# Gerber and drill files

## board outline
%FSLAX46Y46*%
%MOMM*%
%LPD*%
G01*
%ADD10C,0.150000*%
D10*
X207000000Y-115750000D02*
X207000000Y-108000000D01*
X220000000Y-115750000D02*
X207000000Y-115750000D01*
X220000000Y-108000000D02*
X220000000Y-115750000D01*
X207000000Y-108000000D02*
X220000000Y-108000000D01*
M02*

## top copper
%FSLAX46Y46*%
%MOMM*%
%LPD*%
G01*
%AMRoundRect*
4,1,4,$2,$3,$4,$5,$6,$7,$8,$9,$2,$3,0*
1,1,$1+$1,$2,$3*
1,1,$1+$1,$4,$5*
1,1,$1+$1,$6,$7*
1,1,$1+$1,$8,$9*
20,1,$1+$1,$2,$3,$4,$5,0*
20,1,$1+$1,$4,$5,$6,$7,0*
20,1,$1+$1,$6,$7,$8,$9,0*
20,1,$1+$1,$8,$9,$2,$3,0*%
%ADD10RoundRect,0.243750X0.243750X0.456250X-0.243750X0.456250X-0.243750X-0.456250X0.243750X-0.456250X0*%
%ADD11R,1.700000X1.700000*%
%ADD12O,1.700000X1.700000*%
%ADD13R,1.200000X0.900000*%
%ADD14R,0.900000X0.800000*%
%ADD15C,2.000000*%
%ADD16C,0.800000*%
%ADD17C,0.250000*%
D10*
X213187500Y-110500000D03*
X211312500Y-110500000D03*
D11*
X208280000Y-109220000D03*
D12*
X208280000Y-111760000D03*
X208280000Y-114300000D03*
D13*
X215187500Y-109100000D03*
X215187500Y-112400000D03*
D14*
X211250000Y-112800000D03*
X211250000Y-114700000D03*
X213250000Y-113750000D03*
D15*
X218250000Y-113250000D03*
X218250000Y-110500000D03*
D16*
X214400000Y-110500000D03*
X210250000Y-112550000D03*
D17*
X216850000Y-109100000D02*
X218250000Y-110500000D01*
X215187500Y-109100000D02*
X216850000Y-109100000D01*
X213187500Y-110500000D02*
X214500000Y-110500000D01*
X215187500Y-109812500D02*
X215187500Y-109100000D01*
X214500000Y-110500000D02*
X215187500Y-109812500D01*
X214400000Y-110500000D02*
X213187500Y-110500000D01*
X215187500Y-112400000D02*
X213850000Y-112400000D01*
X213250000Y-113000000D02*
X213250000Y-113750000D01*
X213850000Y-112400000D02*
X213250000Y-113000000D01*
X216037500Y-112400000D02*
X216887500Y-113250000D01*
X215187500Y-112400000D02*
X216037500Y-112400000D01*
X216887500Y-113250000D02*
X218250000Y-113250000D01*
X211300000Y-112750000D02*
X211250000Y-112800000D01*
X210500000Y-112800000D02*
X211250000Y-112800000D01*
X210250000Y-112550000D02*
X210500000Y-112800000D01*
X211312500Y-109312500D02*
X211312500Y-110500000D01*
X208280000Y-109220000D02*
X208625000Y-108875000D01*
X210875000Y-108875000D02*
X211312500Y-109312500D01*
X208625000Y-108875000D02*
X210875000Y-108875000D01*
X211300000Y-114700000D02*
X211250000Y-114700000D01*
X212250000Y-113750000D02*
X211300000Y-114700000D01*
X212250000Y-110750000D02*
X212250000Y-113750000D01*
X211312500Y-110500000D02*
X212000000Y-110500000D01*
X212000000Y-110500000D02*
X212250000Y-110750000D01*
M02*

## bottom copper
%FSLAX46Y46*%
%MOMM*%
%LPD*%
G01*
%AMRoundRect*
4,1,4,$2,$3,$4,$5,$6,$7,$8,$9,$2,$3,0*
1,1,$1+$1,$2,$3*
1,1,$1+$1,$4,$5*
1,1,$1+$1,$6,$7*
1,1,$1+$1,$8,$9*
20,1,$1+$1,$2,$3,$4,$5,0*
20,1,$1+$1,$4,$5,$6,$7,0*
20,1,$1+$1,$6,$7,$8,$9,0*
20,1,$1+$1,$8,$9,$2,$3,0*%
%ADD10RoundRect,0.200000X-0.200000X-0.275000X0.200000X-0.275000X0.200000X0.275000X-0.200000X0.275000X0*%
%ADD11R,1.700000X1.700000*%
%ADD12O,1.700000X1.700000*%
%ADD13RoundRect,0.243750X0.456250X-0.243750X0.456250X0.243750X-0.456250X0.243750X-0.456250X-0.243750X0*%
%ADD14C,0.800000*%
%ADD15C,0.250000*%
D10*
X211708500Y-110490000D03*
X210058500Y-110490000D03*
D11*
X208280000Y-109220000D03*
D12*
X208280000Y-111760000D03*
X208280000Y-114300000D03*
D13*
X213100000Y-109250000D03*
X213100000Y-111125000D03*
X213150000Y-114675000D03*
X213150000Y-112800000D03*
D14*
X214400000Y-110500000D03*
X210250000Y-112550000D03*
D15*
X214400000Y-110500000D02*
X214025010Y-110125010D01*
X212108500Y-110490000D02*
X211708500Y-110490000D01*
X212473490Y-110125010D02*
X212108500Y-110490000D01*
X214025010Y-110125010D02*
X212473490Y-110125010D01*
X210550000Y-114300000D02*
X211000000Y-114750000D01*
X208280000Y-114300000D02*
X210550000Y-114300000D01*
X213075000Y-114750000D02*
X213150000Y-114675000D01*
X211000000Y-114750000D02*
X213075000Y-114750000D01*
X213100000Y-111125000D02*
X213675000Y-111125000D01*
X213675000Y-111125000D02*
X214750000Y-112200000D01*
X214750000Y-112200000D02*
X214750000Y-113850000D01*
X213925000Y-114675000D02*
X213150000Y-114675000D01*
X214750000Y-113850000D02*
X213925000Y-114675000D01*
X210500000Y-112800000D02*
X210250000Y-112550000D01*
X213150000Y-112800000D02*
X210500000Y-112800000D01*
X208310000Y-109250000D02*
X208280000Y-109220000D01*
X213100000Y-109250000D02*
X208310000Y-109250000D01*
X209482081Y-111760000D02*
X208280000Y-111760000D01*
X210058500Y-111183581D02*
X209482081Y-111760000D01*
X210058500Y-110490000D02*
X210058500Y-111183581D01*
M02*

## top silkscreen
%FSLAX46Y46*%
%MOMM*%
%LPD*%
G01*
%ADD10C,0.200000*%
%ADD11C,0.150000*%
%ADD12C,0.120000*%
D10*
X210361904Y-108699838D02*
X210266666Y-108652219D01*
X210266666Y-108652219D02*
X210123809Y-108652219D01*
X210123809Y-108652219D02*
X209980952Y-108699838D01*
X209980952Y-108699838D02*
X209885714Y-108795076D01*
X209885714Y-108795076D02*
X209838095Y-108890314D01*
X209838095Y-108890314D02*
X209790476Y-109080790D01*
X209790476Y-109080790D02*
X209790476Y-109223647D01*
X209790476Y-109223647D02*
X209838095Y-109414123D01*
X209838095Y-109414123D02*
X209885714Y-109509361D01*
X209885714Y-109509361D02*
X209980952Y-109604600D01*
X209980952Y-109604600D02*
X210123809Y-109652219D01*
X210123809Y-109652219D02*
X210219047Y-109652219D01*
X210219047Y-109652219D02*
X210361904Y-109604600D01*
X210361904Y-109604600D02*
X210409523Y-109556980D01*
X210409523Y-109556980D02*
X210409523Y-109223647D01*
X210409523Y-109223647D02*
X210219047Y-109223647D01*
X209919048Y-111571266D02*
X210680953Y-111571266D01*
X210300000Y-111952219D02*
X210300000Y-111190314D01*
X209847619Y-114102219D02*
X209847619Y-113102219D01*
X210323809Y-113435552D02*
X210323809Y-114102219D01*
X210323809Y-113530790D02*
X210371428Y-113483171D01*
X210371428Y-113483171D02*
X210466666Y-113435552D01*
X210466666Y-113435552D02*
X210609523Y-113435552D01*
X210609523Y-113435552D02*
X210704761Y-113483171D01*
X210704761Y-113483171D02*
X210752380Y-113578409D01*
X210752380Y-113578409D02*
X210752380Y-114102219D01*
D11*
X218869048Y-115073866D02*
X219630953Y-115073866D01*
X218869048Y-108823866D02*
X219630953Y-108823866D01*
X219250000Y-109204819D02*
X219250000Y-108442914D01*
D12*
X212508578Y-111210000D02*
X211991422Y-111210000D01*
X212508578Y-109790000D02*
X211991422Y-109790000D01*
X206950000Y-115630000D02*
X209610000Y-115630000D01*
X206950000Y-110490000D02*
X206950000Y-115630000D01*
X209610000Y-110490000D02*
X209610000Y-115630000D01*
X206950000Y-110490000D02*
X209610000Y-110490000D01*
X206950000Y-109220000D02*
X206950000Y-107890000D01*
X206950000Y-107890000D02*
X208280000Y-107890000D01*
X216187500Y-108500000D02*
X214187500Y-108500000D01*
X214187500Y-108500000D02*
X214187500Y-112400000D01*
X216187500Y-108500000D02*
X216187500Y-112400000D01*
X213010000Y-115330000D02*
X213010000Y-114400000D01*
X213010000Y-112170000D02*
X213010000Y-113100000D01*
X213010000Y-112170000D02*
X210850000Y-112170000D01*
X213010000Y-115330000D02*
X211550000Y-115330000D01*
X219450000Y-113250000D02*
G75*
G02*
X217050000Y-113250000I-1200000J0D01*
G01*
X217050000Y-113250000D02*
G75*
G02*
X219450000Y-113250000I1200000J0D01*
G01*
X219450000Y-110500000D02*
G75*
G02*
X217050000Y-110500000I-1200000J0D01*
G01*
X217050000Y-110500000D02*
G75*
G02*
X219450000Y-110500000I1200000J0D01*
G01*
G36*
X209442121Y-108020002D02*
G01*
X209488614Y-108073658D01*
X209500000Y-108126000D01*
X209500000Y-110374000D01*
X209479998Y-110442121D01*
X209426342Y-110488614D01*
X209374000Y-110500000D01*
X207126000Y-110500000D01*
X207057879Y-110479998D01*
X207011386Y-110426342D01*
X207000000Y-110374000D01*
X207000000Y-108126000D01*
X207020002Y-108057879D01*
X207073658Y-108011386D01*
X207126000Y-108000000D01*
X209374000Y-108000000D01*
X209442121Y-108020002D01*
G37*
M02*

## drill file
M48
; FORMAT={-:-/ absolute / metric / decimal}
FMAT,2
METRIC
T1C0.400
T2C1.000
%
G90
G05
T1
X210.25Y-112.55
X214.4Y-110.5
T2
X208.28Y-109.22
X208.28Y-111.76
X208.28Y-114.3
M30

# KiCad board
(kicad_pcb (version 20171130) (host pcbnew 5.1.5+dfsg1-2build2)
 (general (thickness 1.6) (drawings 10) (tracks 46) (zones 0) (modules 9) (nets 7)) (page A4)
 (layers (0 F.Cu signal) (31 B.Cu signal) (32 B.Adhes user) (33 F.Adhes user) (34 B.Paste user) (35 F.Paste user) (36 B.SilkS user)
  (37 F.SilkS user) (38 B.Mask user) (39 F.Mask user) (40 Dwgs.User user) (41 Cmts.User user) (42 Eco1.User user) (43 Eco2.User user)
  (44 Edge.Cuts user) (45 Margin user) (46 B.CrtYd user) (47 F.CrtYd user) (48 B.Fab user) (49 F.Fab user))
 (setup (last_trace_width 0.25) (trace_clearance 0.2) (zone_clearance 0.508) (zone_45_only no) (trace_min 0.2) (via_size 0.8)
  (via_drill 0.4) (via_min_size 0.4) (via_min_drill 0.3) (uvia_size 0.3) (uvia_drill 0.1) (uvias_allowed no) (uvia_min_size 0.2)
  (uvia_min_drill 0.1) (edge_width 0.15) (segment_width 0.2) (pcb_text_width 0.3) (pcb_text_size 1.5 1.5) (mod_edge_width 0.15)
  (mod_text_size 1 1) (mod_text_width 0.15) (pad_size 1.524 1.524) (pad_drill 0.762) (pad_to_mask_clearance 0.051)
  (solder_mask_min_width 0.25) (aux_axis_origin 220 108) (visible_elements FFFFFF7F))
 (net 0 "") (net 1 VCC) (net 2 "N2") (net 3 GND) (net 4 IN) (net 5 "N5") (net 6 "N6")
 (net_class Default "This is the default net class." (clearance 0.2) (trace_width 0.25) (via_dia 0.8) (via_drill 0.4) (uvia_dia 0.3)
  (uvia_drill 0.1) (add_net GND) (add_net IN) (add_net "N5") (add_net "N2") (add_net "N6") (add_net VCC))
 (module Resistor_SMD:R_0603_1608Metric (layer B.Cu) (at 210.8835 110.49)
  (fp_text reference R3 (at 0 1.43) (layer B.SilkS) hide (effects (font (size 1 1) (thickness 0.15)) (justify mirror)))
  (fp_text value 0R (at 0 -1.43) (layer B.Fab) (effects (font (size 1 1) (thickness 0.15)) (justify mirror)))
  (pad 2 smd roundrect (at 0.825 0) (size 0.8 0.95) (layers B.Cu B.Paste B.Mask) (roundrect_rratio 0.25) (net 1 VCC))
  (pad 1 smd roundrect (at -0.825 0) (size 0.8 0.95) (layers B.Cu B.Paste B.Mask) (roundrect_rratio 0.25) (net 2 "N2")))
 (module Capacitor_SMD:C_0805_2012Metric (layer F.Cu) (at 212.25 110.5 180)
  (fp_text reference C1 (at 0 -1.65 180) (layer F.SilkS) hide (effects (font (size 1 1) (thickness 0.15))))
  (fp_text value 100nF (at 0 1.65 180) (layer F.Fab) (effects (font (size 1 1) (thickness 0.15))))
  (fp_line (start -0.258578 -0.71) (end 0.258578 -0.71) (layer F.SilkS) (width 0.12))
  (fp_line (start -0.258578 0.71) (end 0.258578 0.71) (layer F.SilkS) (width 0.12))
  (pad 1 smd roundrect (at -0.9375 0 180) (size 0.975 1.4) (layers F.Cu F.Paste F.Mask) (roundrect_rratio 0.25) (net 1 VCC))
  (pad 2 smd roundrect (at 0.9375 0 180) (size 0.975 1.4) (layers F.Cu F.Paste F.Mask) (roundrect_rratio 0.25) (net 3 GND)))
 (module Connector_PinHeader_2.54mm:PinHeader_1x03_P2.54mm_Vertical (layer F.Cu) (at 208.28 109.22)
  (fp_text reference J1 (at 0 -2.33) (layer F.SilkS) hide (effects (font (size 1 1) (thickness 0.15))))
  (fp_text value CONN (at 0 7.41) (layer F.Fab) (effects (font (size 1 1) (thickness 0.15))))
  (fp_line (start -1.33 6.41) (end 1.33 6.41) (layer F.SilkS) (width 0.12))
  (fp_line (start -1.33 1.27) (end -1.33 6.41) (layer F.SilkS) (width 0.12))
  (fp_line (start 1.33 1.27) (end 1.33 6.41) (layer F.SilkS) (width 0.12))
  (fp_line (start -1.33 1.27) (end 1.33 1.27) (layer F.SilkS) (width 0.12))
  (fp_line (start -1.33 0) (end -1.33 -1.33) (layer F.SilkS) (width 0.12))
  (fp_line (start -1.33 -1.33) (end 0 -1.33) (layer F.SilkS) (width 0.12))
  (pad 1 thru_hole rect (at 0 0) (size 1.7 1.7) (drill 1) (layers *.Cu *.Mask) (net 3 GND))
  (pad 2 thru_hole oval (at 0 2.54) (size 1.7 1.7) (drill 1) (layers *.Cu *.Mask) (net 2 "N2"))
  (pad 3 thru_hole oval (at 0 5.08) (size 1.7 1.7) (drill 1) (layers *.Cu *.Mask) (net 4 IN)))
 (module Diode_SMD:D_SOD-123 (layer F.Cu) (at 215.1875 110.75 270)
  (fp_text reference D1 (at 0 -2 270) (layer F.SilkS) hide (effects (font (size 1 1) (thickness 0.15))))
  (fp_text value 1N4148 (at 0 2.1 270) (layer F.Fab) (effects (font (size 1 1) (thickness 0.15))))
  (fp_line (start -2.25 -1) (end -2.25 1) (layer F.SilkS) (width 0.12))
  (fp_line (start -2.25 1) (end 1.65 1) (layer F.SilkS) (width 0.12))
  (fp_line (start -2.25 -1) (end 1.65 -1) (layer F.SilkS) (width 0.12))
  (pad 1 smd rect (at -1.65 0 270) (size 0.9 1.2) (layers F.Cu F.Paste F.Mask) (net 1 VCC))
  (pad 2 smd rect (at 1.65 0 270) (size 0.9 1.2) (layers F.Cu F.Paste F.Mask) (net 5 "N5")))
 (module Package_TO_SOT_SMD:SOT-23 (layer F.Cu) (at 212.25 113.75)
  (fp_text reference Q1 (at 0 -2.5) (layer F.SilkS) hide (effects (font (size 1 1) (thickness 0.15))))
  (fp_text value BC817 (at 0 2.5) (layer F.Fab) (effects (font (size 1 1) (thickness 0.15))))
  (fp_line (start 0.76 1.58) (end 0.76 0.65) (layer F.SilkS) (width 0.12))
  (fp_line (start 0.76 -1.58) (end 0.76 -0.65) (layer F.SilkS) (width 0.12))
  (fp_line (start 0.76 -1.58) (end -1.4 -1.58) (layer F.SilkS) (width 0.12))
  (fp_line (start 0.76 1.58) (end -0.7 1.58) (layer F.SilkS) (width 0.12))
  (pad 1 smd rect (at -1 -0.95) (size 0.9 0.8) (layers F.Cu F.Paste F.Mask) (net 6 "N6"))
  (pad 2 smd rect (at -1 0.95) (size 0.9 0.8) (layers F.Cu F.Paste F.Mask) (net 3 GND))
  (pad 3 smd rect (at 1 0) (size 0.9 0.8) (layers F.Cu F.Paste F.Mask) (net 5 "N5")))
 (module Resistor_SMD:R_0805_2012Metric (layer B.Cu) (at 213.1 110.1875 90)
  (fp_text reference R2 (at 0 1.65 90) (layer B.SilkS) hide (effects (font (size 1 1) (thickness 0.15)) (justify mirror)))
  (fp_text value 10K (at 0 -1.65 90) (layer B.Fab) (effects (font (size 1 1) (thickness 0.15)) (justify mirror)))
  (pad 2 smd roundrect (at 0.9375 0 90) (size 0.975 1.4) (layers B.Cu B.Paste B.Mask) (roundrect_rratio 0.25) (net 3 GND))
  (pad 1 smd roundrect (at -0.9375 0 90) (size 0.975 1.4) (layers B.Cu B.Paste B.Mask) (roundrect_rratio 0.25) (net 4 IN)))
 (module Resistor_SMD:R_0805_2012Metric (layer B.Cu) (at 213.15 113.7375 90)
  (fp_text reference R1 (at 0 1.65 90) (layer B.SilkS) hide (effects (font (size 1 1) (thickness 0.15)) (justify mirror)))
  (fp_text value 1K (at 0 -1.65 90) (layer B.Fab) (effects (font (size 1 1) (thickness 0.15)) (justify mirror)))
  (pad 1 smd roundrect (at -0.9375 0 90) (size 0.975 1.4) (layers B.Cu B.Paste B.Mask) (roundrect_rratio 0.25) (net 4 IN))
  (pad 2 smd roundrect (at 0.9375 0 90) (size 0.975 1.4) (layers B.Cu B.Paste B.Mask) (roundrect_rratio 0.25) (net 6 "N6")))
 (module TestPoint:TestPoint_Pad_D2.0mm (layer F.Cu) (at 218.25 113.25)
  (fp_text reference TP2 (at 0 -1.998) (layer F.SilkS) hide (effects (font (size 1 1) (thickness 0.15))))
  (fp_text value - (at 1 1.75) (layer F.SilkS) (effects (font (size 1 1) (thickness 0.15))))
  (fp_circle (center 0 0) (end 0 1.2) (layer F.SilkS) (width 0.12))
  (pad 1 smd circle (at 0 0) (size 2 2) (layers F.Cu F.Mask) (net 5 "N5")))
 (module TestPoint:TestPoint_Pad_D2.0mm (layer F.Cu) (at 218.25 110.5)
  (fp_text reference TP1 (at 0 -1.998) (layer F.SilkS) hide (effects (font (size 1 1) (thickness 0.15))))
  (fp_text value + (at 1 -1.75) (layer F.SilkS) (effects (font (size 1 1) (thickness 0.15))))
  (fp_circle (center 0 0) (end 0 1.2) (layer F.SilkS) (width 0.12))
  (pad 1 smd circle (at 0 0) (size 2 2) (layers F.Cu F.Mask) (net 1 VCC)))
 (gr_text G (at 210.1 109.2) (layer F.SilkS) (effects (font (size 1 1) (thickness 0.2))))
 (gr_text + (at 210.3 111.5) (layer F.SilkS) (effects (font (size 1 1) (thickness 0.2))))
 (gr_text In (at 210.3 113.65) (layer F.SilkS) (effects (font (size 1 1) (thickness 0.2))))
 (gr_line (start 207 115.75) (end 207 108) (layer Edge.Cuts) (width 0.15))
 (gr_line (start 220 115.75) (end 207 115.75) (layer Edge.Cuts) (width 0.15))
 (gr_line (start 220 108) (end 220 115.75) (layer Edge.Cuts) (width 0.15))
 (gr_line (start 207 108) (end 220 108) (layer Edge.Cuts) (width 0.15))
 (segment (start 216.85 109.1) (end 218.25 110.5) (width 0.25) (layer F.Cu) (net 1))
 (segment (start 215.1875 109.1) (end 216.85 109.1) (width 0.25) (layer F.Cu) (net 1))
 (segment (start 213.1875 110.5) (end 214.5 110.5) (width 0.25) (layer F.Cu) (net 1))
 (segment (start 215.1875 109.8125) (end 215.1875 109.1) (width 0.25) (layer F.Cu) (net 1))
 (segment (start 214.5 110.5) (end 215.1875 109.8125) (width 0.25) (layer F.Cu) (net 1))
 (segment (start 214.4 110.5) (end 213.1875 110.5) (width 0.25) (layer F.Cu) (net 1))
 (via (at 214.4 110.5) (size 0.8) (drill 0.4) (layers F.Cu B.Cu) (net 1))
 (segment (start 214.4 110.5) (end 214.02501 110.12501) (width 0.25) (layer B.Cu) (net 1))
 (segment (start 212.1085 110.49) (end 211.7085 110.49) (width 0.25) (layer B.Cu) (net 1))
 (segment (start 212.47349 110.12501) (end 212.1085 110.49) (width 0.25) (layer B.Cu) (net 1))
 (segment (start 214.02501 110.12501) (end 212.47349 110.12501) (width 0.25) (layer B.Cu) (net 1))
 (segment (start 215.1875 112.4) (end 213.85 112.4) (width 0.25) (layer F.Cu) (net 5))
 (segment (start 213.25 113) (end 213.25 113.75) (width 0.25) (layer F.Cu) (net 5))
 (segment (start 213.85 112.4) (end 213.25 113) (width 0.25) (layer F.Cu) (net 5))
 (segment (start 216.0375 112.4) (end 216.8875 113.25) (width 0.25) (layer F.Cu) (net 5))
 (segment (start 215.1875 112.4) (end 216.0375 112.4) (width 0.25) (layer F.Cu) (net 5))
 (segment (start 216.8875 113.25) (end 218.25 113.25) (width 0.25) (layer F.Cu) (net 5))
 (segment (start 210.55 114.3) (end 211 114.75) (width 0.25) (layer B.Cu) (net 4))
 (segment (start 208.28 114.3) (end 210.55 114.3) (width 0.25) (layer B.Cu) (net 4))
 (segment (start 213.075 114.75) (end 213.15 114.675) (width 0.25) (layer B.Cu) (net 4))
 (segment (start 211 114.75) (end 213.075 114.75) (width 0.25) (layer B.Cu) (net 4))
 (segment (start 213.1 111.125) (end 213.675 111.125) (width 0.25) (layer B.Cu) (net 4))
 (segment (start 213.675 111.125) (end 214.75 112.2) (width 0.25) (layer B.Cu) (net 4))
 (segment (start 214.75 112.2) (end 214.75 113.85) (width 0.25) (layer B.Cu) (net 4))
 (segment (start 213.925 114.675) (end 213.15 114.675) (width 0.25) (layer B.Cu) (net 4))
 (segment (start 214.75 113.85) (end 213.925 114.675) (width 0.25) (layer B.Cu) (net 4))
 (segment (start 211.3 112.75) (end 211.25 112.8) (width 0.25) (layer F.Cu) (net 6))
 (via (at 210.25 112.55) (size 0.8) (drill 0.4) (layers F.Cu B.Cu) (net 6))
 (segment (start 210.5 112.8) (end 210.25 112.55) (width 0.25) (layer B.Cu) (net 6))
 (segment (start 213.15 112.8) (end 210.5 112.8) (width 0.25) (layer B.Cu) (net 6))
 (segment (start 210.5 112.8) (end 211.25 112.8) (width 0.25) (layer F.Cu) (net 6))
 (segment (start 210.25 112.55) (end 210.5 112.8) (width 0.25) (layer F.Cu) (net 6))
 (segment (start 211.3125 109.3125) (end 211.3125 110.5) (width 0.25) (layer F.Cu) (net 3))
 (segment (start 208.28 109.22) (end 208.625 108.875) (width 0.25) (layer F.Cu) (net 3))
 (segment (start 210.875 108.875) (end 211.3125 109.3125) (width 0.25) (layer F.Cu) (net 3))
 (segment (start 208.625 108.875) (end 210.875 108.875) (width 0.25) (layer F.Cu) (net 3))
 (segment (start 211.3 114.7) (end 211.25 114.7) (width 0.25) (layer F.Cu) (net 3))
 (segment (start 212.25 113.75) (end 211.3 114.7) (width 0.25) (layer F.Cu) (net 3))
 (segment (start 212.25 110.75) (end 212.25 113.75) (width 0.25) (layer F.Cu) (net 3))
 (segment (start 211.3125 110.5) (end 212 110.5) (width 0.25) (layer F.Cu) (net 3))
 (segment (start 212 110.5) (end 212.25 110.75) (width 0.25) (layer F.Cu) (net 3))
 (segment (start 208.31 109.25) (end 208.28 109.22) (width 0.25) (layer B.Cu) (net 3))
 (segment (start 213.1 109.25) (end 208.31 109.25) (width 0.25) (layer B.Cu) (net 3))
 (segment (start 209.482081 111.76) (end 208.28 111.76) (width 0.25) (layer B.Cu) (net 2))
 (segment (start 210.0585 111.183581) (end 209.482081 111.76) (width 0.25) (layer B.Cu) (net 2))
 (segment (start 210.0585 110.49) (end 210.0585 111.183581) (width 0.25) (layer B.Cu) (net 2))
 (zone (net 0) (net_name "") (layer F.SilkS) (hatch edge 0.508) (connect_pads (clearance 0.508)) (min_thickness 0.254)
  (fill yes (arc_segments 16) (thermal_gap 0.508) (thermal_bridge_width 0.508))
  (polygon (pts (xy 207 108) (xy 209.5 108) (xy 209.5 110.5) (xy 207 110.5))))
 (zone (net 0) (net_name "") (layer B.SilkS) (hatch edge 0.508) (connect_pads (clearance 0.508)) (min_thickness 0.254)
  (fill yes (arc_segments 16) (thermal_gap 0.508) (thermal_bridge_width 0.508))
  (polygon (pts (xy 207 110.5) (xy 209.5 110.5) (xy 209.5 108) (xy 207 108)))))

